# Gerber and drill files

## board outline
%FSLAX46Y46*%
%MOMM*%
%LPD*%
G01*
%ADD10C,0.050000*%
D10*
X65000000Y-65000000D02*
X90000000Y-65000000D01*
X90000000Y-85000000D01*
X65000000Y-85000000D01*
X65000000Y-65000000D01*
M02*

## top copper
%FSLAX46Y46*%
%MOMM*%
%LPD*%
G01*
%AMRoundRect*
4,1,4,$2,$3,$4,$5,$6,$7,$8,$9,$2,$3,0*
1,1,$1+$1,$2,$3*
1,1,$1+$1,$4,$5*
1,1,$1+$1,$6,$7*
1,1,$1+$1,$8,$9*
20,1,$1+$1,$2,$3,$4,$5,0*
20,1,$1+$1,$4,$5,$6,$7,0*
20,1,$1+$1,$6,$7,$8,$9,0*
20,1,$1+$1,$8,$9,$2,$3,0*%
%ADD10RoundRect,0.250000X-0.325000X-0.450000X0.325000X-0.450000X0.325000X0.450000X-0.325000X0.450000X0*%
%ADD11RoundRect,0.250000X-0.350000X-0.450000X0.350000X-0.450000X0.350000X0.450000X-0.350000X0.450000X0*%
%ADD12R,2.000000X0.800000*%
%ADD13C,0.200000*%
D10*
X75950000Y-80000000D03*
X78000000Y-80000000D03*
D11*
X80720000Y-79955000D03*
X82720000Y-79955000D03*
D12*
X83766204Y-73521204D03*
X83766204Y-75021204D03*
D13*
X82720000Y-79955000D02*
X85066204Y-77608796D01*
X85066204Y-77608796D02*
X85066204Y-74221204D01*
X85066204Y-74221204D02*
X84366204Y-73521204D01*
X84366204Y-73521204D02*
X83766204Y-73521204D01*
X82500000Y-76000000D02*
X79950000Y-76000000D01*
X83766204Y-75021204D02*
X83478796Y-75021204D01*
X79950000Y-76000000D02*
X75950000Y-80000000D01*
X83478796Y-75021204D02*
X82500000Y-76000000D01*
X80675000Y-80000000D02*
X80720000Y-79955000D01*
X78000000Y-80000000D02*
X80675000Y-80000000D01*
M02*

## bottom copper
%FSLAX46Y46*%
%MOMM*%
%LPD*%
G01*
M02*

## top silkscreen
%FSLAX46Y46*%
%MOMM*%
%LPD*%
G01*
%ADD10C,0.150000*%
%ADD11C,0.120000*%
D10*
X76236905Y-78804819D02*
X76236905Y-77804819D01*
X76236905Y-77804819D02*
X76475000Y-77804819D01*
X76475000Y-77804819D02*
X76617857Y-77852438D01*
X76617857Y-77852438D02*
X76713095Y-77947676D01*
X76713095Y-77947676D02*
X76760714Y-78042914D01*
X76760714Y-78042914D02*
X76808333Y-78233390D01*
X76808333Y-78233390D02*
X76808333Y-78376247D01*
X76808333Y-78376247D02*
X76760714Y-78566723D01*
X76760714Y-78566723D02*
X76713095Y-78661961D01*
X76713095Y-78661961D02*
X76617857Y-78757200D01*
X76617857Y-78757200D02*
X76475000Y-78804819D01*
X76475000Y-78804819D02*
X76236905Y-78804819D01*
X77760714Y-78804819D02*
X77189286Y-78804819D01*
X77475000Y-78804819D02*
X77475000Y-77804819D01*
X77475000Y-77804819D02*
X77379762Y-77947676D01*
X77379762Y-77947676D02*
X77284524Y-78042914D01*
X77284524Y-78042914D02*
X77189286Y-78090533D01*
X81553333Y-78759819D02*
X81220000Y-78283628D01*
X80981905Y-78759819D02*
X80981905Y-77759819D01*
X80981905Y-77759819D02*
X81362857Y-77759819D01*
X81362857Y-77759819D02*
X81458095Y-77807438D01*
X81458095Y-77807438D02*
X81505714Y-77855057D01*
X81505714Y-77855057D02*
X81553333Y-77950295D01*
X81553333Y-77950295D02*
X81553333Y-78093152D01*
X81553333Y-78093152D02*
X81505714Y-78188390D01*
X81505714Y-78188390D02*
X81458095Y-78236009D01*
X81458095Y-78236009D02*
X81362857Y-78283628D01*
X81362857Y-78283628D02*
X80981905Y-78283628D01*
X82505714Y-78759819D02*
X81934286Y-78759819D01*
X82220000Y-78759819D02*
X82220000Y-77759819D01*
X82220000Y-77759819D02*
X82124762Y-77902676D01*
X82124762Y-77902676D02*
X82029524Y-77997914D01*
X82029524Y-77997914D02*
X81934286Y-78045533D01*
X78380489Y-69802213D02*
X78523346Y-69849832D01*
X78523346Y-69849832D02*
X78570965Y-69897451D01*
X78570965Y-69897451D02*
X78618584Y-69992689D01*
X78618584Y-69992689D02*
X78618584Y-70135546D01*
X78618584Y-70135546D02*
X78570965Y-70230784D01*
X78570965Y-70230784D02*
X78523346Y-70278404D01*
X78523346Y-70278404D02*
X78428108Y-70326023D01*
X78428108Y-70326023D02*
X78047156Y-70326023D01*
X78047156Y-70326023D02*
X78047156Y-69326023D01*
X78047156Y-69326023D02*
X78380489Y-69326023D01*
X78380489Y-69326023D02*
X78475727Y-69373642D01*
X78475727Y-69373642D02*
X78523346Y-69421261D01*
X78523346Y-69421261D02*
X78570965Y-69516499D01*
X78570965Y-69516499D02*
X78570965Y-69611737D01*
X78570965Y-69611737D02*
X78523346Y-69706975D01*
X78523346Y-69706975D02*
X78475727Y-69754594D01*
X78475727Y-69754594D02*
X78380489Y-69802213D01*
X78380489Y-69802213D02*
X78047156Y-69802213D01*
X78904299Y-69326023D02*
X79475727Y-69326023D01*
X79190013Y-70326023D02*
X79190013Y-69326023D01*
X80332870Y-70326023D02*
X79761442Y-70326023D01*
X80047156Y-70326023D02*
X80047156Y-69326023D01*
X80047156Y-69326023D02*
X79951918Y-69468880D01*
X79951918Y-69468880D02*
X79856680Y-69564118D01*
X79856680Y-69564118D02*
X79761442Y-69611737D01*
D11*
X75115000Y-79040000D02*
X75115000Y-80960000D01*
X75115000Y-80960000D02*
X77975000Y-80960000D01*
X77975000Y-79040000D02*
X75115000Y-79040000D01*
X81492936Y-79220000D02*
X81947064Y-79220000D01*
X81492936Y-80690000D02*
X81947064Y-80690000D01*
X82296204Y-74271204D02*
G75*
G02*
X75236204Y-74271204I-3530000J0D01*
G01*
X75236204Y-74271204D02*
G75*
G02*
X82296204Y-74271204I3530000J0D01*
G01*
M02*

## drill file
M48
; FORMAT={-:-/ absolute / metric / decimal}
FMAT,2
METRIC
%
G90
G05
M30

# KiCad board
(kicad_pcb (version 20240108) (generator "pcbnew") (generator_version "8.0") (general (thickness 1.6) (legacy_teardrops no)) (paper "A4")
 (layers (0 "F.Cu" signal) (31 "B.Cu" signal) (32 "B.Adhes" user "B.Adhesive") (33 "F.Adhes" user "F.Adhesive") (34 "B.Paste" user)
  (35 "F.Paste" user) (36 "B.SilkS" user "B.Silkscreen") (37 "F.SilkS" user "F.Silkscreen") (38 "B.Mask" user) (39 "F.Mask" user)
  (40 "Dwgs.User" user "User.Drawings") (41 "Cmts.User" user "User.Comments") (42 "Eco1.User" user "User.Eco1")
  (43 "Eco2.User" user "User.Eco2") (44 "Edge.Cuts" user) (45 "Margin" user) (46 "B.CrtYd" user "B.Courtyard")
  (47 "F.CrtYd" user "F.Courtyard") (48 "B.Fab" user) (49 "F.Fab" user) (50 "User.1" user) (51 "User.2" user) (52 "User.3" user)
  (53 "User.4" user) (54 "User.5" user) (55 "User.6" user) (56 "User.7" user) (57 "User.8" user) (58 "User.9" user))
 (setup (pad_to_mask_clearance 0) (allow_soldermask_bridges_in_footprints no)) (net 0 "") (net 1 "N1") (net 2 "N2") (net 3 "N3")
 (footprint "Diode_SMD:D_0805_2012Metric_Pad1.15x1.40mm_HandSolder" (layer "F.Cu") (at 76.975 80)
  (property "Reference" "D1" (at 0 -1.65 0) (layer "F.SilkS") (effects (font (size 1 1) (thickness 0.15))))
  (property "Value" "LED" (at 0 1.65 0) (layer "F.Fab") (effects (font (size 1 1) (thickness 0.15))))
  (fp_line (start -1.86 -0.96) (end -1.86 0.96) (stroke (width 0.12) (type solid)) (layer "F.SilkS"))
  (fp_line (start -1.86 0.96) (end 1 0.96) (stroke (width 0.12) (type solid)) (layer "F.SilkS"))
  (fp_line (start 1 -0.96) (end -1.86 -0.96) (stroke (width 0.12) (type solid)) (layer "F.SilkS"))
  (pad "1" smd roundrect (at -1.025 0) (size 1.15 1.4) (layers "F.Cu" "F.Paste" "F.Mask") (roundrect_rratio 0.217391) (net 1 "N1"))
  (pad "2" smd roundrect (at 1.025 0) (size 1.15 1.4) (layers "F.Cu" "F.Paste" "F.Mask") (roundrect_rratio 0.217391) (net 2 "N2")))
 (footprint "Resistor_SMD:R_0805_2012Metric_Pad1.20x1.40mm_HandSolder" (layer "F.Cu") (at 81.72 79.955)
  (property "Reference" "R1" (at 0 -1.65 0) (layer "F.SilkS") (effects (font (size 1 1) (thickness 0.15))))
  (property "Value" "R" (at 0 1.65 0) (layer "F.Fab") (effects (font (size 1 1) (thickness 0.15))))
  (fp_line (start -0.227064 -0.735) (end 0.227064 -0.735) (stroke (width 0.12) (type solid)) (layer "F.SilkS"))
  (fp_line (start -0.227064 0.735) (end 0.227064 0.735) (stroke (width 0.12) (type solid)) (layer "F.SilkS"))
  (pad "1" smd roundrect (at -1 0) (size 1.2 1.4) (layers "F.Cu" "F.Paste" "F.Mask") (roundrect_rratio 0.208333) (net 2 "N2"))
  (pad "2" smd roundrect (at 1 0) (size 1.2 1.4) (layers "F.Cu" "F.Paste" "F.Mask") (roundrect_rratio 0.208333) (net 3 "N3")))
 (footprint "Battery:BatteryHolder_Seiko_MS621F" (layer "F.Cu") (at 83.766204 74.271204)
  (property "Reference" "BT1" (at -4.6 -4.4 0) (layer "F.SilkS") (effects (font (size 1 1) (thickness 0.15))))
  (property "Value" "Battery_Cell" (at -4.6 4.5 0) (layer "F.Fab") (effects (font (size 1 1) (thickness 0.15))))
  (fp_circle (center -5 0) (end -1.47 0) (stroke (width 0.12) (type solid)) (fill none) (layer "F.SilkS"))
  (pad "1" smd rect (at 0 -0.75) (size 2 0.8) (layers "F.Cu" "F.Paste" "F.Mask") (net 3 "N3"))
  (pad "2" smd rect (at 0 0.75) (size 2 0.8) (layers "F.Cu" "F.Paste" "F.Mask") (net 1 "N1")))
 (gr_rect (start 65 65) (end 90 85) (stroke (width 0.05) (type default)) (fill none) (layer "Edge.Cuts"))
 (segment (start 82.72 79.955) (end 85.066204 77.608796) (width 0.2) (layer "F.Cu") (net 3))
 (segment (start 85.066204 77.608796) (end 85.066204 74.221204) (width 0.2) (layer "F.Cu") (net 3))
 (segment (start 85.066204 74.221204) (end 84.366204 73.521204) (width 0.2) (layer "F.Cu") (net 3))
 (segment (start 84.366204 73.521204) (end 83.766204 73.521204) (width 0.2) (layer "F.Cu") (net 3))
 (segment (start 82.5 76) (end 79.95 76) (width 0.2) (layer "F.Cu") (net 1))
 (segment (start 83.766204 75.021204) (end 83.478796 75.021204) (width 0.2) (layer "F.Cu") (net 1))
 (segment (start 79.95 76) (end 75.95 80) (width 0.2) (layer "F.Cu") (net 1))
 (segment (start 83.478796 75.021204) (end 82.5 76) (width 0.2) (layer "F.Cu") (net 1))
 (segment (start 80.675 80) (end 80.72 79.955) (width 0.2) (layer "F.Cu") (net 2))
 (segment (start 78 80) (end 80.675 80) (width 0.2) (layer "F.Cu") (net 2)))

